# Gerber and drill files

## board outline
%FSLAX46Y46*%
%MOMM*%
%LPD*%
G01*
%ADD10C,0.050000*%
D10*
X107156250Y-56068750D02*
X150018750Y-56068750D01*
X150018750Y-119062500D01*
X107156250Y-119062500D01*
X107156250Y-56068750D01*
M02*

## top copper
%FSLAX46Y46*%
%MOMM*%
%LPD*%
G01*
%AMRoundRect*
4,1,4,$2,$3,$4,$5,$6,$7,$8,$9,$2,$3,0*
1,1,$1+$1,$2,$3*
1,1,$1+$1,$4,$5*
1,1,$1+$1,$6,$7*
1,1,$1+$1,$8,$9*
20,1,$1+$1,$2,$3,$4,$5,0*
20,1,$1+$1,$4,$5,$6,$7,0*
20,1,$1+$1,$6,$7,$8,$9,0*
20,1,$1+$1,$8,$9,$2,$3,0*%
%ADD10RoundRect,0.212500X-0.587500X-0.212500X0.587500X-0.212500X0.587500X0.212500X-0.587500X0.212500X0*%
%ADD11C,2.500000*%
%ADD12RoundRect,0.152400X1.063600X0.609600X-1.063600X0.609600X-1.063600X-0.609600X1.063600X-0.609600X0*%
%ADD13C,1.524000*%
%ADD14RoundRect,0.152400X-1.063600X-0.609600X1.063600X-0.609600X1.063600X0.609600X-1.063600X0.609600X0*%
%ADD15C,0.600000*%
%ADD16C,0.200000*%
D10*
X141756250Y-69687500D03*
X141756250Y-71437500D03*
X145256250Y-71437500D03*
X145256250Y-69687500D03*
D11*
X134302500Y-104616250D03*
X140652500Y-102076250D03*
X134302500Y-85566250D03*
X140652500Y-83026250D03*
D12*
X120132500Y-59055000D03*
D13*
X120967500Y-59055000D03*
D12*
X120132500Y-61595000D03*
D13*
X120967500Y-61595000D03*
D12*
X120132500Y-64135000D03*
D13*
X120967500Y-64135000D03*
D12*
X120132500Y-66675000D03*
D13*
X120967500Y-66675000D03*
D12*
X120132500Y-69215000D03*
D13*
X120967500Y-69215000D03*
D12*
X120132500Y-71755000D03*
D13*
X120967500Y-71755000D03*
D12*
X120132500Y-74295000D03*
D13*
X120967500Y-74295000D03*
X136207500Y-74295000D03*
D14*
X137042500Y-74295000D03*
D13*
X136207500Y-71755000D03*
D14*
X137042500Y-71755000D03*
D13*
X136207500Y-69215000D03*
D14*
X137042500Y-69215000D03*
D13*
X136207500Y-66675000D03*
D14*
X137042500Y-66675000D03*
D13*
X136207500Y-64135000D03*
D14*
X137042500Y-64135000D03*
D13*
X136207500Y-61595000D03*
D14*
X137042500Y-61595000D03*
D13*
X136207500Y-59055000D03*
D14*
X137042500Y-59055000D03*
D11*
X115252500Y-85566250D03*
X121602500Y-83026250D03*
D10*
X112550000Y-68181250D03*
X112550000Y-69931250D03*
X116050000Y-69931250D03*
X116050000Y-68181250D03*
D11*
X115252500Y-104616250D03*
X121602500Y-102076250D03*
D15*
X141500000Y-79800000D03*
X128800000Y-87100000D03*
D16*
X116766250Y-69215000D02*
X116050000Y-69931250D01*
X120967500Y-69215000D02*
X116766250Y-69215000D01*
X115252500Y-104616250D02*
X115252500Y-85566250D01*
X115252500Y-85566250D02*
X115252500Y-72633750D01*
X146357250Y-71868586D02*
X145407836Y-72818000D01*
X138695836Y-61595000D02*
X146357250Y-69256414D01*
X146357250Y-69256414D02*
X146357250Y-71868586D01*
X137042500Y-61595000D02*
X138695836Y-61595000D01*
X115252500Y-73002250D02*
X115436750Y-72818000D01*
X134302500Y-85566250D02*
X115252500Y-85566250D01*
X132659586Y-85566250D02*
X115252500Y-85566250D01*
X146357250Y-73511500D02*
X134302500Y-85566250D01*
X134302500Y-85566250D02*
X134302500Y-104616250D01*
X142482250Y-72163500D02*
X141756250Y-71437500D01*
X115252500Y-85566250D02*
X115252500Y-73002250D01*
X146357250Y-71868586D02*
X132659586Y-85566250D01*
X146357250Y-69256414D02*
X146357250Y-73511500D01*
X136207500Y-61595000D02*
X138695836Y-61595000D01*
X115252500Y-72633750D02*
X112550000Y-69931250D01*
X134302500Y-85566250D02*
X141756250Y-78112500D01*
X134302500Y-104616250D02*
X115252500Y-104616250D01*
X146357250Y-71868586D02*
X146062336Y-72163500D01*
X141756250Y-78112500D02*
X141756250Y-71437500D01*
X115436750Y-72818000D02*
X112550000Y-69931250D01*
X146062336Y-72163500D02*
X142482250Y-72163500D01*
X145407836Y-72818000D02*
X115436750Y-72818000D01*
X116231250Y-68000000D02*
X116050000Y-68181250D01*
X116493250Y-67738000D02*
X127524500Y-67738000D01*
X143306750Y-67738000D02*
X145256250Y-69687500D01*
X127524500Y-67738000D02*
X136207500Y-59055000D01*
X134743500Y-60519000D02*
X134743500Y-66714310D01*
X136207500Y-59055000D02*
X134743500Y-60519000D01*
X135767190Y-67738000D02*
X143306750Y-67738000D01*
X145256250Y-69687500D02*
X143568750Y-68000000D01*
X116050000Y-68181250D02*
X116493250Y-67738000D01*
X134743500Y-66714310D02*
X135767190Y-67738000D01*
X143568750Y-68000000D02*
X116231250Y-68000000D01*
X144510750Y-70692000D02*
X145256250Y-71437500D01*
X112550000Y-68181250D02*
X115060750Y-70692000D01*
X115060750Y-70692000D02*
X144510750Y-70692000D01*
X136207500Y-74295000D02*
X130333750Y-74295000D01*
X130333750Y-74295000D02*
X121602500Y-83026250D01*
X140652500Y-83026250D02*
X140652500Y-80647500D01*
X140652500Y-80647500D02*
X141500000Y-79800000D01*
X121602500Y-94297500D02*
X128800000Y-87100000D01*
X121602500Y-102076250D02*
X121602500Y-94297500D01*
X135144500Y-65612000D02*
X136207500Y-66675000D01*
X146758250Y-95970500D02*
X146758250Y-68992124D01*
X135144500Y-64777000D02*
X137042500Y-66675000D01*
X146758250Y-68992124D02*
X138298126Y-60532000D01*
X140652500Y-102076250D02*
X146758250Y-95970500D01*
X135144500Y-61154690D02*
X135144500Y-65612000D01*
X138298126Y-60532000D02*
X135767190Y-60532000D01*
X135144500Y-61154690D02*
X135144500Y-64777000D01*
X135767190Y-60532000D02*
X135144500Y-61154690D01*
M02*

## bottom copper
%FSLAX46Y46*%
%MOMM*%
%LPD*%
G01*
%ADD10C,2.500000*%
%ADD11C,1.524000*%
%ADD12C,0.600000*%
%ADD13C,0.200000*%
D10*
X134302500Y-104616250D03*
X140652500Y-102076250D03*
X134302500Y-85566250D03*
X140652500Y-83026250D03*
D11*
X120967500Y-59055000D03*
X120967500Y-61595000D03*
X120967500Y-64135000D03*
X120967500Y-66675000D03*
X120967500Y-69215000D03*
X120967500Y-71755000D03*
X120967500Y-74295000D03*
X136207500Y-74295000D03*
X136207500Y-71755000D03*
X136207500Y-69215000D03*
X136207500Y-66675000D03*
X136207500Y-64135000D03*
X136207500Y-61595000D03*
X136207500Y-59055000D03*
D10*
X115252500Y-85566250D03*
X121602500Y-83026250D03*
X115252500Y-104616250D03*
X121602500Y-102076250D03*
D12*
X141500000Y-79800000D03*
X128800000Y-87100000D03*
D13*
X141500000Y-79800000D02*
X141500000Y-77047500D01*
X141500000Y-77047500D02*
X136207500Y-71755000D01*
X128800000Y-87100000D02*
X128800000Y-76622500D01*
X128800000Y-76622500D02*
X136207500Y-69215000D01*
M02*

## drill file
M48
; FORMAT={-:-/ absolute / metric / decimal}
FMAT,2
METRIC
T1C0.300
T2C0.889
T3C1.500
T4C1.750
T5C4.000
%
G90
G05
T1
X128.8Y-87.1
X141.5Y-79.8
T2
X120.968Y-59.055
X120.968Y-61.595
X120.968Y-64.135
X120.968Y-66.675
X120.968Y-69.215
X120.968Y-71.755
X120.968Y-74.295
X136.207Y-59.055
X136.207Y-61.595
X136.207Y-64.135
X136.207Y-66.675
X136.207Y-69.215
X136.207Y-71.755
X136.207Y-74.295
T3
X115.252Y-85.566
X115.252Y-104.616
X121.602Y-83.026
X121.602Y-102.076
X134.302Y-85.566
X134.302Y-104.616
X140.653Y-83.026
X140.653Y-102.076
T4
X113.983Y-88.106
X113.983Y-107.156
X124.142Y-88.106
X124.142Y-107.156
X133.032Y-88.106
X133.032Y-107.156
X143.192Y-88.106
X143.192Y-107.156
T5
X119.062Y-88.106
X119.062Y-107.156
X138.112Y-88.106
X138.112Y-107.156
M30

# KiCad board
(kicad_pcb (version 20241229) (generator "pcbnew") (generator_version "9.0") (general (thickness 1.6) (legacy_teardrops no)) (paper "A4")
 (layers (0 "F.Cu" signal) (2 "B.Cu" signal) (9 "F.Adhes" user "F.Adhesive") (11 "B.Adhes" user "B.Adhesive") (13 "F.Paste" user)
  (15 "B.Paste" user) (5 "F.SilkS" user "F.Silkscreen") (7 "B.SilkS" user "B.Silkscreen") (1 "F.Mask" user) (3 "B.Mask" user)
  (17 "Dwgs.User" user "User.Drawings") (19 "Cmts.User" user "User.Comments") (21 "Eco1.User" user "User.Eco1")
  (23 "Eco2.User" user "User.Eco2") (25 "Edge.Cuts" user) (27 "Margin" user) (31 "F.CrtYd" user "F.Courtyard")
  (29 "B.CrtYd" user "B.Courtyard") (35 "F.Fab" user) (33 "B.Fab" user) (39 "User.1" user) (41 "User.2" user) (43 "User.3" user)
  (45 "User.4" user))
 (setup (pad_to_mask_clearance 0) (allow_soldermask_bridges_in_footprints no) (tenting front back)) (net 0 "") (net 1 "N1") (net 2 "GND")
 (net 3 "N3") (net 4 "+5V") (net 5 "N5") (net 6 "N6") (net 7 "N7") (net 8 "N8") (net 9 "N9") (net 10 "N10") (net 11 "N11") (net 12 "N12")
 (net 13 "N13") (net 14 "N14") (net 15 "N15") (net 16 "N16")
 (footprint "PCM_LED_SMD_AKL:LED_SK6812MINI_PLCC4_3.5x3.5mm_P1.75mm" (layer "F.Cu") (at 143.50625 70.5625)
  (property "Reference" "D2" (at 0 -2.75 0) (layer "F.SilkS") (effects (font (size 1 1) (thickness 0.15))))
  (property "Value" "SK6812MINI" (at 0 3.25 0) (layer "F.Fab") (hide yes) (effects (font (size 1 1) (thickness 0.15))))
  (pad "1" smd roundrect (at -1.75 -0.875) (size 1.6 0.85) (layers "F.Cu" "F.Mask" "F.Paste") (roundrect_rratio 0.25) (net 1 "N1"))
  (pad "2" smd roundrect (at -1.75 0.875) (size 1.6 0.85) (layers "F.Cu" "F.Mask" "F.Paste") (roundrect_rratio 0.25) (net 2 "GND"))
  (pad "3" smd roundrect (at 1.75 0.875) (size 1.6 0.85) (layers "F.Cu" "F.Mask" "F.Paste") (roundrect_rratio 0.25) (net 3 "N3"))
  (pad "4" smd roundrect (at 1.75 -0.875) (size 1.6 0.85) (layers "F.Cu" "F.Mask" "F.Paste") (roundrect_rratio 0.25) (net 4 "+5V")))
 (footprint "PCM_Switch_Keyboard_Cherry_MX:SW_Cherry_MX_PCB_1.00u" (layer "F.Cu") (at 138.1125 107.15625)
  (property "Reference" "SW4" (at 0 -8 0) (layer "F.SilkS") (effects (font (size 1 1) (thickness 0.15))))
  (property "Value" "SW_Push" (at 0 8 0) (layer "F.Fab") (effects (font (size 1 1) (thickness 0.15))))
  (pad "" np_thru_hole circle (at -5.08 0) (size 1.75 1.75) (drill 1.75) (layers "*.Cu" "*.Mask"))
  (pad "" np_thru_hole circle (at 0 0) (size 4 4) (drill 4) (layers "*.Cu" "*.Mask"))
  (pad "" np_thru_hole circle (at 5.08 0) (size 1.75 1.75) (drill 1.75) (layers "*.Cu" "*.Mask"))
  (pad "1" thru_hole circle (at -3.81 -2.54) (size 2.5 2.5) (drill 1.5) (layers "*.Cu" "*.Mask") (remove_unused_layers no) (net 2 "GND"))
  (pad "2" thru_hole circle (at 2.54 -5.08) (size 2.5 2.5) (drill 1.5) (layers "*.Cu" "*.Mask") (remove_unused_layers no) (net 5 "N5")))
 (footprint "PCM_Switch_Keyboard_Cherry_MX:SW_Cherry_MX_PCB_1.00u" (layer "F.Cu") (at 138.1125 88.10625)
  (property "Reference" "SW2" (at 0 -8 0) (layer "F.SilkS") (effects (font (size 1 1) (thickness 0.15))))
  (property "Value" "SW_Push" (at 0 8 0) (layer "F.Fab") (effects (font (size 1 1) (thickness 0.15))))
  (pad "" np_thru_hole circle (at -5.08 0) (size 1.75 1.75) (drill 1.75) (layers "*.Cu" "*.Mask"))
  (pad "" np_thru_hole circle (at 0 0) (size 4 4) (drill 4) (layers "*.Cu" "*.Mask"))
  (pad "" np_thru_hole circle (at 5.08 0) (size 1.75 1.75) (drill 1.75) (layers "*.Cu" "*.Mask"))
  (pad "1" thru_hole circle (at -3.81 -2.54) (size 2.5 2.5) (drill 1.5) (layers "*.Cu" "*.Mask") (remove_unused_layers no) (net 2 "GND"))
  (pad "2" thru_hole circle (at 2.54 -5.08) (size 2.5 2.5) (drill 1.5) (layers "*.Cu" "*.Mask") (remove_unused_layers no) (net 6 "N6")))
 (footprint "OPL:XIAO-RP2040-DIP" (layer "F.Cu") (at 128.5875 66.675)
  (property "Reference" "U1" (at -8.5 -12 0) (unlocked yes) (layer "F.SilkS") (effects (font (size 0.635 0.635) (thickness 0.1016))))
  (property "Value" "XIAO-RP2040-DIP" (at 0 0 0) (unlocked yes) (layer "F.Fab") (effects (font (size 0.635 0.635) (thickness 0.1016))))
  (pad "1" smd roundrect (at -8.455 -7.62 180) (size 2.432 1.524) (layers "F.Cu" "F.Mask") (roundrect_rratio 0.1) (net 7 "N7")
   (thermal_bridge_angle 45))
  (pad "1" thru_hole circle (at -7.62 -7.62 180) (size 1.524 1.524) (drill 0.889) (layers "*.Cu" "*.Mask") (remove_unused_layers no)
   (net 7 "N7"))
  (pad "2" smd roundrect (at -8.455 -5.08 180) (size 2.432 1.524) (layers "F.Cu" "F.Mask") (roundrect_rratio 0.1) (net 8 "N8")
   (thermal_bridge_angle 45))
  (pad "2" thru_hole circle (at -7.62 -5.08 180) (size 1.524 1.524) (drill 0.889) (layers "*.Cu" "*.Mask") (remove_unused_layers no)
   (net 8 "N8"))
  (pad "3" smd roundrect (at -8.455 -2.54 180) (size 2.432 1.524) (layers "F.Cu" "F.Mask") (roundrect_rratio 0.1) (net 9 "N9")
   (thermal_bridge_angle 45))
  (pad "3" thru_hole circle (at -7.62 -2.54 180) (size 1.524 1.524) (drill 0.889) (layers "*.Cu" "*.Mask") (remove_unused_layers no)
   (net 9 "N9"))
  (pad "4" smd roundrect (at -8.455 0 180) (size 2.432 1.524) (layers "F.Cu" "F.Mask") (roundrect_rratio 0.1) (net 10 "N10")
   (thermal_bridge_angle 45))
  (pad "4" thru_hole circle (at -7.62 0 180) (size 1.524 1.524) (drill 0.889) (layers "*.Cu" "*.Mask") (remove_unused_layers no)
   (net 10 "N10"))
  (pad "5" smd roundrect (at -8.455 2.54 180) (size 2.432 1.524) (layers "F.Cu" "F.Mask") (roundrect_rratio 0.1) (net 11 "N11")
   (thermal_bridge_angle 45))
  (pad "5" thru_hole circle (at -7.62 2.54 180) (size 1.524 1.524) (drill 0.889) (layers "*.Cu" "*.Mask") (remove_unused_layers no)
   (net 11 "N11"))
  (pad "6" smd roundrect (at -8.455 5.08 180) (size 2.432 1.524) (layers "F.Cu" "F.Mask") (roundrect_rratio 0.1) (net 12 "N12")
   (thermal_bridge_angle 45))
  (pad "6" thru_hole circle (at -7.62 5.08 180) (size 1.524 1.524) (drill 0.889) (layers "*.Cu" "*.Mask") (remove_unused_layers no)
   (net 12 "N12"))
  (pad "7" smd roundrect (at -8.455 7.62 180) (size 2.432 1.524) (layers "F.Cu" "F.Mask") (roundrect_rratio 0.1) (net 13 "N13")
   (thermal_bridge_angle 45))
  (pad "7" thru_hole circle (at -7.62 7.62 180) (size 1.524 1.524) (drill 0.889) (layers "*.Cu" "*.Mask") (remove_unused_layers no)
   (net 13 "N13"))
  (pad "8" thru_hole circle (at 7.62 7.62) (size 1.524 1.524) (drill 0.889) (layers "*.Cu" "*.Mask") (remove_unused_layers no)
   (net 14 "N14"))
  (pad "8" smd roundrect (at 8.455 7.62) (size 2.432 1.524) (layers "F.Cu" "F.Mask") (roundrect_rratio 0.1) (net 14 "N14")
   (thermal_bridge_angle 45))
  (pad "9" thru_hole circle (at 7.62 5.08) (size 1.524 1.524) (drill 0.889) (layers "*.Cu" "*.Mask") (remove_unused_layers no) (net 6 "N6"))
  (pad "9" smd roundrect (at 8.455 5.08) (size 2.432 1.524) (layers "F.Cu" "F.Mask") (roundrect_rratio 0.1) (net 6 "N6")
   (thermal_bridge_angle 45))
  (pad "10" thru_hole circle (at 7.62 2.54) (size 1.524 1.524) (drill 0.889) (layers "*.Cu" "*.Mask") (remove_unused_layers no)
   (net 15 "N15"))
  (pad "10" smd roundrect (at 8.455 2.54) (size 2.432 1.524) (layers "F.Cu" "F.Mask") (roundrect_rratio 0.1) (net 15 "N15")
   (thermal_bridge_angle 45))
  (pad "11" thru_hole circle (at 7.62 0) (size 1.524 1.524) (drill 0.889) (layers "*.Cu" "*.Mask") (remove_unused_layers no) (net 5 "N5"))
  (pad "11" smd roundrect (at 8.455 0) (size 2.432 1.524) (layers "F.Cu" "F.Mask") (roundrect_rratio 0.1) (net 5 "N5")
   (thermal_bridge_angle 45))
  (pad "12" thru_hole circle (at 7.62 -2.54) (size 1.524 1.524) (drill 0.889) (layers "*.Cu" "*.Mask") (remove_unused_layers no)
   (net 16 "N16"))
  (pad "12" smd roundrect (at 8.455 -2.54) (size 2.432 1.524) (layers "F.Cu" "F.Mask") (roundrect_rratio 0.1) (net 16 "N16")
   (thermal_bridge_angle 45))
  (pad "13" thru_hole circle (at 7.62 -5.08) (size 1.524 1.524) (drill 0.889) (layers "*.Cu" "*.Mask") (remove_unused_layers no)
   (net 2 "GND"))
  (pad "13" smd roundrect (at 8.455 -5.08) (size 2.432 1.524) (layers "F.Cu" "F.Mask") (roundrect_rratio 0.1) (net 2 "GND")
   (thermal_bridge_angle 45))
  (pad "14" thru_hole circle (at 7.62 -7.62) (size 1.524 1.524) (drill 0.889) (layers "*.Cu" "*.Mask") (remove_unused_layers no)
   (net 4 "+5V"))
  (pad "14" smd roundrect (at 8.455 -7.62) (size 2.432 1.524) (layers "F.Cu" "F.Mask") (roundrect_rratio 0.1) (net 4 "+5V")
   (thermal_bridge_angle 45)))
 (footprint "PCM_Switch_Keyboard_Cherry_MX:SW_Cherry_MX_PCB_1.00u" (layer "F.Cu") (at 119.0625 88.10625)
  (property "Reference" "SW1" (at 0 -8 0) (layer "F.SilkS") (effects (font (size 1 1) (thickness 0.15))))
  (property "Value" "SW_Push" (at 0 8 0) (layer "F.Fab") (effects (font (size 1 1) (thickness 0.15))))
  (pad "" np_thru_hole circle (at -5.08 0) (size 1.75 1.75) (drill 1.75) (layers "*.Cu" "*.Mask"))
  (pad "" np_thru_hole circle (at 0 0) (size 4 4) (drill 4) (layers "*.Cu" "*.Mask"))
  (pad "" np_thru_hole circle (at 5.08 0) (size 1.75 1.75) (drill 1.75) (layers "*.Cu" "*.Mask"))
  (pad "1" thru_hole circle (at -3.81 -2.54) (size 2.5 2.5) (drill 1.5) (layers "*.Cu" "*.Mask") (remove_unused_layers no) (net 2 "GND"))
  (pad "2" thru_hole circle (at 2.54 -5.08) (size 2.5 2.5) (drill 1.5) (layers "*.Cu" "*.Mask") (remove_unused_layers no) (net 14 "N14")))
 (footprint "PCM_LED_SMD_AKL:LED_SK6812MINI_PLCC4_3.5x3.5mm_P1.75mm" (layer "F.Cu") (at 114.3 69.05625)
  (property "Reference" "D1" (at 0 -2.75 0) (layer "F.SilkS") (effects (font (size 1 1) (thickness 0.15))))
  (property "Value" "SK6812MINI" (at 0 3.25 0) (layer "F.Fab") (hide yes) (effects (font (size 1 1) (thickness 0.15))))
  (pad "1" smd roundrect (at -1.75 -0.875) (size 1.6 0.85) (layers "F.Cu" "F.Mask" "F.Paste") (roundrect_rratio 0.25) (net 3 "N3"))
  (pad "2" smd roundrect (at -1.75 0.875) (size 1.6 0.85) (layers "F.Cu" "F.Mask" "F.Paste") (roundrect_rratio 0.25) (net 2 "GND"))
  (pad "3" smd roundrect (at 1.75 0.875) (size 1.6 0.85) (layers "F.Cu" "F.Mask" "F.Paste") (roundrect_rratio 0.25) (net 11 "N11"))
  (pad "4" smd roundrect (at 1.75 -0.875) (size 1.6 0.85) (layers "F.Cu" "F.Mask" "F.Paste") (roundrect_rratio 0.25) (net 4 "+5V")))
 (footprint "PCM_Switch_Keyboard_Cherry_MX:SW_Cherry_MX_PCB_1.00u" (layer "F.Cu") (at 119.0625 107.15625)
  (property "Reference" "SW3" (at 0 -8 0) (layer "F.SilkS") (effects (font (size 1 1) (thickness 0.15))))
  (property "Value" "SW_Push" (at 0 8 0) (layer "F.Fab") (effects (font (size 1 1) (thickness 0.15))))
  (pad "" np_thru_hole circle (at -5.08 0) (size 1.75 1.75) (drill 1.75) (layers "*.Cu" "*.Mask"))
  (pad "" np_thru_hole circle (at 0 0) (size 4 4) (drill 4) (layers "*.Cu" "*.Mask"))
  (pad "" np_thru_hole circle (at 5.08 0) (size 1.75 1.75) (drill 1.75) (layers "*.Cu" "*.Mask"))
  (pad "1" thru_hole circle (at -3.81 -2.54) (size 2.5 2.5) (drill 1.5) (layers "*.Cu" "*.Mask") (remove_unused_layers no) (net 2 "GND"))
  (pad "2" thru_hole circle (at 2.54 -5.08) (size 2.5 2.5) (drill 1.5) (layers "*.Cu" "*.Mask") (remove_unused_layers no) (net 15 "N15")))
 (gr_rect (start 107.15625 56.06875) (end 150.01875 119.0625) (stroke (width 0.05) (type default)) (fill no) (layer "Edge.Cuts"))
 (segment (start 116.76625 69.215) (end 116.05 69.93125) (width 0.2) (layer "F.Cu") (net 11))
 (segment (start 120.9675 69.215) (end 116.76625 69.215) (width 0.2) (layer "F.Cu") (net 11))
 (segment (start 115.2525 104.61625) (end 115.2525 85.56625) (width 0.2) (layer "F.Cu") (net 2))
 (segment (start 115.2525 85.56625) (end 115.2525 72.63375) (width 0.2) (layer "F.Cu") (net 2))
 (segment (start 146.35725 71.868586) (end 145.407836 72.818) (width 0.2) (layer "F.Cu") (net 2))
 (segment (start 138.695836 61.595) (end 146.35725 69.256414) (width 0.2) (layer "F.Cu") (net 2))
 (segment (start 146.35725 69.256414) (end 146.35725 71.868586) (width 0.2) (layer "F.Cu") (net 2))
 (segment (start 137.0425 61.595) (end 138.695836 61.595) (width 0.2) (layer "F.Cu") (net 2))
 (segment (start 115.2525 73.00225) (end 115.43675 72.818) (width 0.2) (layer "F.Cu") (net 2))
 (segment (start 134.3025 85.56625) (end 115.2525 85.56625) (width 0.2) (layer "F.Cu") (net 2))
 (segment (start 132.659586 85.56625) (end 115.2525 85.56625) (width 0.2) (layer "F.Cu") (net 2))
 (segment (start 146.35725 73.5115) (end 134.3025 85.56625) (width 0.2) (layer "F.Cu") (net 2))
 (segment (start 134.3025 85.56625) (end 134.3025 104.61625) (width 0.2) (layer "F.Cu") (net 2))
 (segment (start 142.48225 72.1635) (end 141.75625 71.4375) (width 0.2) (layer "F.Cu") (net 2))
 (segment (start 115.2525 85.56625) (end 115.2525 73.00225) (width 0.2) (layer "F.Cu") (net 2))
 (segment (start 146.35725 71.868586) (end 132.659586 85.56625) (width 0.2) (layer "F.Cu") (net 2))
 (segment (start 146.35725 69.256414) (end 146.35725 73.5115) (width 0.2) (layer "F.Cu") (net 2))
 (segment (start 136.2075 61.595) (end 138.695836 61.595) (width 0.2) (layer "F.Cu") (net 2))
 (segment (start 115.2525 72.63375) (end 112.55 69.93125) (width 0.2) (layer "F.Cu") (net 2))
 (segment (start 134.3025 85.56625) (end 141.75625 78.1125) (width 0.2) (layer "F.Cu") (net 2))
 (segment (start 134.3025 104.61625) (end 115.2525 104.61625) (width 0.2) (layer "F.Cu") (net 2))
 (segment (start 146.35725 71.868586) (end 146.062336 72.1635) (width 0.2) (layer "F.Cu") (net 2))
 (segment (start 141.75625 78.1125) (end 141.75625 71.4375) (width 0.2) (layer "F.Cu") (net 2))
 (segment (start 115.43675 72.818) (end 112.55 69.93125) (width 0.2) (layer "F.Cu") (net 2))
 (segment (start 146.062336 72.1635) (end 142.48225 72.1635) (width 0.2) (layer "F.Cu") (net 2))
 (segment (start 145.407836 72.818) (end 115.43675 72.818) (width 0.2) (layer "F.Cu") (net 2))
 (segment (start 116.23125 68) (end 116.05 68.18125) (width 0.2) (layer "F.Cu") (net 4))
 (segment (start 116.49325 67.738) (end 127.5245 67.738) (width 0.2) (layer "F.Cu") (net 4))
 (segment (start 143.30675 67.738) (end 145.25625 69.6875) (width 0.2) (layer "F.Cu") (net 4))
 (segment (start 127.5245 67.738) (end 136.2075 59.055) (width 0.2) (layer "F.Cu") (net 4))
 (segment (start 134.7435 60.519) (end 134.7435 66.71431) (width 0.2) (layer "F.Cu") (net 4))
 (segment (start 136.2075 59.055) (end 134.7435 60.519) (width 0.2) (layer "F.Cu") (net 4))
 (segment (start 135.76719 67.738) (end 143.30675 67.738) (width 0.2) (layer "F.Cu") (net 4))
 (segment (start 145.25625 69.6875) (end 143.56875 68) (width 0.2) (layer "F.Cu") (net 4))
 (segment (start 116.05 68.18125) (end 116.49325 67.738) (width 0.2) (layer "F.Cu") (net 4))
 (segment (start 134.7435 66.71431) (end 135.76719 67.738) (width 0.2) (layer "F.Cu") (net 4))
 (segment (start 143.56875 68) (end 116.23125 68) (width 0.2) (layer "F.Cu") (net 4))
 (segment (start 144.51075 70.692) (end 145.25625 71.4375) (width 0.2) (layer "F.Cu") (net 3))
 (segment (start 112.55 68.18125) (end 115.06075 70.692) (width 0.2) (layer "F.Cu") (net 3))
 (segment (start 115.06075 70.692) (end 144.51075 70.692) (width 0.2) (layer "F.Cu") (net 3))
 (segment (start 136.2075 74.295) (end 130.33375 74.295) (width 0.2) (layer "F.Cu") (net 14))
 (segment (start 130.33375 74.295) (end 121.6025 83.02625) (width 0.2) (layer "F.Cu") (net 14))
 (segment (start 140.6525 83.02625) (end 140.6525 80.6475) (width 0.2) (layer "F.Cu") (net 6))
 (segment (start 140.6525 80.6475) (end 141.5 79.8) (width 0.2) (layer "F.Cu") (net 6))
 (via (at 141.5 79.8) (size 0.6) (drill 0.3) (layers "F.Cu" "B.Cu") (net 6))
 (segment (start 141.5 79.8) (end 141.5 77.0475) (width 0.2) (layer "B.Cu") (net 6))
 (segment (start 141.5 77.0475) (end 136.2075 71.755) (width 0.2) (layer "B.Cu") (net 6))
 (segment (start 121.6025 94.2975) (end 128.8 87.1) (width 0.2) (layer "F.Cu") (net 15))
 (segment (start 121.6025 102.07625) (end 121.6025 94.2975) (width 0.2) (layer "F.Cu") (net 15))
 (via (at 128.8 87.1) (size 0.6) (drill 0.3) (layers "F.Cu" "B.Cu") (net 15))
 (segment (start 128.8 87.1) (end 128.8 76.6225) (width 0.2) (layer "B.Cu") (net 15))
 (segment (start 128.8 76.6225) (end 136.2075 69.215) (width 0.2) (layer "B.Cu") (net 15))
 (segment (start 135.1445 65.612) (end 136.2075 66.675) (width 0.2) (layer "F.Cu") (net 5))
 (segment (start 146.75825 95.9705) (end 146.75825 68.992124) (width 0.2) (layer "F.Cu") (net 5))
 (segment (start 135.1445 64.777) (end 137.0425 66.675) (width 0.2) (layer "F.Cu") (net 5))
 (segment (start 146.75825 68.992124) (end 138.298126 60.532) (width 0.2) (layer "F.Cu") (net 5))
 (segment (start 140.6525 102.07625) (end 146.75825 95.9705) (width 0.2) (layer "F.Cu") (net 5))
 (segment (start 135.1445 61.15469) (end 135.1445 65.612) (width 0.2) (layer "F.Cu") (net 5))
 (segment (start 138.298126 60.532) (end 135.76719 60.532) (width 0.2) (layer "F.Cu") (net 5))
 (segment (start 135.1445 61.15469) (end 135.1445 64.777) (width 0.2) (layer "F.Cu") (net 5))
 (segment (start 135.76719 60.532) (end 135.1445 61.15469) (width 0.2) (layer "F.Cu") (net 5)))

